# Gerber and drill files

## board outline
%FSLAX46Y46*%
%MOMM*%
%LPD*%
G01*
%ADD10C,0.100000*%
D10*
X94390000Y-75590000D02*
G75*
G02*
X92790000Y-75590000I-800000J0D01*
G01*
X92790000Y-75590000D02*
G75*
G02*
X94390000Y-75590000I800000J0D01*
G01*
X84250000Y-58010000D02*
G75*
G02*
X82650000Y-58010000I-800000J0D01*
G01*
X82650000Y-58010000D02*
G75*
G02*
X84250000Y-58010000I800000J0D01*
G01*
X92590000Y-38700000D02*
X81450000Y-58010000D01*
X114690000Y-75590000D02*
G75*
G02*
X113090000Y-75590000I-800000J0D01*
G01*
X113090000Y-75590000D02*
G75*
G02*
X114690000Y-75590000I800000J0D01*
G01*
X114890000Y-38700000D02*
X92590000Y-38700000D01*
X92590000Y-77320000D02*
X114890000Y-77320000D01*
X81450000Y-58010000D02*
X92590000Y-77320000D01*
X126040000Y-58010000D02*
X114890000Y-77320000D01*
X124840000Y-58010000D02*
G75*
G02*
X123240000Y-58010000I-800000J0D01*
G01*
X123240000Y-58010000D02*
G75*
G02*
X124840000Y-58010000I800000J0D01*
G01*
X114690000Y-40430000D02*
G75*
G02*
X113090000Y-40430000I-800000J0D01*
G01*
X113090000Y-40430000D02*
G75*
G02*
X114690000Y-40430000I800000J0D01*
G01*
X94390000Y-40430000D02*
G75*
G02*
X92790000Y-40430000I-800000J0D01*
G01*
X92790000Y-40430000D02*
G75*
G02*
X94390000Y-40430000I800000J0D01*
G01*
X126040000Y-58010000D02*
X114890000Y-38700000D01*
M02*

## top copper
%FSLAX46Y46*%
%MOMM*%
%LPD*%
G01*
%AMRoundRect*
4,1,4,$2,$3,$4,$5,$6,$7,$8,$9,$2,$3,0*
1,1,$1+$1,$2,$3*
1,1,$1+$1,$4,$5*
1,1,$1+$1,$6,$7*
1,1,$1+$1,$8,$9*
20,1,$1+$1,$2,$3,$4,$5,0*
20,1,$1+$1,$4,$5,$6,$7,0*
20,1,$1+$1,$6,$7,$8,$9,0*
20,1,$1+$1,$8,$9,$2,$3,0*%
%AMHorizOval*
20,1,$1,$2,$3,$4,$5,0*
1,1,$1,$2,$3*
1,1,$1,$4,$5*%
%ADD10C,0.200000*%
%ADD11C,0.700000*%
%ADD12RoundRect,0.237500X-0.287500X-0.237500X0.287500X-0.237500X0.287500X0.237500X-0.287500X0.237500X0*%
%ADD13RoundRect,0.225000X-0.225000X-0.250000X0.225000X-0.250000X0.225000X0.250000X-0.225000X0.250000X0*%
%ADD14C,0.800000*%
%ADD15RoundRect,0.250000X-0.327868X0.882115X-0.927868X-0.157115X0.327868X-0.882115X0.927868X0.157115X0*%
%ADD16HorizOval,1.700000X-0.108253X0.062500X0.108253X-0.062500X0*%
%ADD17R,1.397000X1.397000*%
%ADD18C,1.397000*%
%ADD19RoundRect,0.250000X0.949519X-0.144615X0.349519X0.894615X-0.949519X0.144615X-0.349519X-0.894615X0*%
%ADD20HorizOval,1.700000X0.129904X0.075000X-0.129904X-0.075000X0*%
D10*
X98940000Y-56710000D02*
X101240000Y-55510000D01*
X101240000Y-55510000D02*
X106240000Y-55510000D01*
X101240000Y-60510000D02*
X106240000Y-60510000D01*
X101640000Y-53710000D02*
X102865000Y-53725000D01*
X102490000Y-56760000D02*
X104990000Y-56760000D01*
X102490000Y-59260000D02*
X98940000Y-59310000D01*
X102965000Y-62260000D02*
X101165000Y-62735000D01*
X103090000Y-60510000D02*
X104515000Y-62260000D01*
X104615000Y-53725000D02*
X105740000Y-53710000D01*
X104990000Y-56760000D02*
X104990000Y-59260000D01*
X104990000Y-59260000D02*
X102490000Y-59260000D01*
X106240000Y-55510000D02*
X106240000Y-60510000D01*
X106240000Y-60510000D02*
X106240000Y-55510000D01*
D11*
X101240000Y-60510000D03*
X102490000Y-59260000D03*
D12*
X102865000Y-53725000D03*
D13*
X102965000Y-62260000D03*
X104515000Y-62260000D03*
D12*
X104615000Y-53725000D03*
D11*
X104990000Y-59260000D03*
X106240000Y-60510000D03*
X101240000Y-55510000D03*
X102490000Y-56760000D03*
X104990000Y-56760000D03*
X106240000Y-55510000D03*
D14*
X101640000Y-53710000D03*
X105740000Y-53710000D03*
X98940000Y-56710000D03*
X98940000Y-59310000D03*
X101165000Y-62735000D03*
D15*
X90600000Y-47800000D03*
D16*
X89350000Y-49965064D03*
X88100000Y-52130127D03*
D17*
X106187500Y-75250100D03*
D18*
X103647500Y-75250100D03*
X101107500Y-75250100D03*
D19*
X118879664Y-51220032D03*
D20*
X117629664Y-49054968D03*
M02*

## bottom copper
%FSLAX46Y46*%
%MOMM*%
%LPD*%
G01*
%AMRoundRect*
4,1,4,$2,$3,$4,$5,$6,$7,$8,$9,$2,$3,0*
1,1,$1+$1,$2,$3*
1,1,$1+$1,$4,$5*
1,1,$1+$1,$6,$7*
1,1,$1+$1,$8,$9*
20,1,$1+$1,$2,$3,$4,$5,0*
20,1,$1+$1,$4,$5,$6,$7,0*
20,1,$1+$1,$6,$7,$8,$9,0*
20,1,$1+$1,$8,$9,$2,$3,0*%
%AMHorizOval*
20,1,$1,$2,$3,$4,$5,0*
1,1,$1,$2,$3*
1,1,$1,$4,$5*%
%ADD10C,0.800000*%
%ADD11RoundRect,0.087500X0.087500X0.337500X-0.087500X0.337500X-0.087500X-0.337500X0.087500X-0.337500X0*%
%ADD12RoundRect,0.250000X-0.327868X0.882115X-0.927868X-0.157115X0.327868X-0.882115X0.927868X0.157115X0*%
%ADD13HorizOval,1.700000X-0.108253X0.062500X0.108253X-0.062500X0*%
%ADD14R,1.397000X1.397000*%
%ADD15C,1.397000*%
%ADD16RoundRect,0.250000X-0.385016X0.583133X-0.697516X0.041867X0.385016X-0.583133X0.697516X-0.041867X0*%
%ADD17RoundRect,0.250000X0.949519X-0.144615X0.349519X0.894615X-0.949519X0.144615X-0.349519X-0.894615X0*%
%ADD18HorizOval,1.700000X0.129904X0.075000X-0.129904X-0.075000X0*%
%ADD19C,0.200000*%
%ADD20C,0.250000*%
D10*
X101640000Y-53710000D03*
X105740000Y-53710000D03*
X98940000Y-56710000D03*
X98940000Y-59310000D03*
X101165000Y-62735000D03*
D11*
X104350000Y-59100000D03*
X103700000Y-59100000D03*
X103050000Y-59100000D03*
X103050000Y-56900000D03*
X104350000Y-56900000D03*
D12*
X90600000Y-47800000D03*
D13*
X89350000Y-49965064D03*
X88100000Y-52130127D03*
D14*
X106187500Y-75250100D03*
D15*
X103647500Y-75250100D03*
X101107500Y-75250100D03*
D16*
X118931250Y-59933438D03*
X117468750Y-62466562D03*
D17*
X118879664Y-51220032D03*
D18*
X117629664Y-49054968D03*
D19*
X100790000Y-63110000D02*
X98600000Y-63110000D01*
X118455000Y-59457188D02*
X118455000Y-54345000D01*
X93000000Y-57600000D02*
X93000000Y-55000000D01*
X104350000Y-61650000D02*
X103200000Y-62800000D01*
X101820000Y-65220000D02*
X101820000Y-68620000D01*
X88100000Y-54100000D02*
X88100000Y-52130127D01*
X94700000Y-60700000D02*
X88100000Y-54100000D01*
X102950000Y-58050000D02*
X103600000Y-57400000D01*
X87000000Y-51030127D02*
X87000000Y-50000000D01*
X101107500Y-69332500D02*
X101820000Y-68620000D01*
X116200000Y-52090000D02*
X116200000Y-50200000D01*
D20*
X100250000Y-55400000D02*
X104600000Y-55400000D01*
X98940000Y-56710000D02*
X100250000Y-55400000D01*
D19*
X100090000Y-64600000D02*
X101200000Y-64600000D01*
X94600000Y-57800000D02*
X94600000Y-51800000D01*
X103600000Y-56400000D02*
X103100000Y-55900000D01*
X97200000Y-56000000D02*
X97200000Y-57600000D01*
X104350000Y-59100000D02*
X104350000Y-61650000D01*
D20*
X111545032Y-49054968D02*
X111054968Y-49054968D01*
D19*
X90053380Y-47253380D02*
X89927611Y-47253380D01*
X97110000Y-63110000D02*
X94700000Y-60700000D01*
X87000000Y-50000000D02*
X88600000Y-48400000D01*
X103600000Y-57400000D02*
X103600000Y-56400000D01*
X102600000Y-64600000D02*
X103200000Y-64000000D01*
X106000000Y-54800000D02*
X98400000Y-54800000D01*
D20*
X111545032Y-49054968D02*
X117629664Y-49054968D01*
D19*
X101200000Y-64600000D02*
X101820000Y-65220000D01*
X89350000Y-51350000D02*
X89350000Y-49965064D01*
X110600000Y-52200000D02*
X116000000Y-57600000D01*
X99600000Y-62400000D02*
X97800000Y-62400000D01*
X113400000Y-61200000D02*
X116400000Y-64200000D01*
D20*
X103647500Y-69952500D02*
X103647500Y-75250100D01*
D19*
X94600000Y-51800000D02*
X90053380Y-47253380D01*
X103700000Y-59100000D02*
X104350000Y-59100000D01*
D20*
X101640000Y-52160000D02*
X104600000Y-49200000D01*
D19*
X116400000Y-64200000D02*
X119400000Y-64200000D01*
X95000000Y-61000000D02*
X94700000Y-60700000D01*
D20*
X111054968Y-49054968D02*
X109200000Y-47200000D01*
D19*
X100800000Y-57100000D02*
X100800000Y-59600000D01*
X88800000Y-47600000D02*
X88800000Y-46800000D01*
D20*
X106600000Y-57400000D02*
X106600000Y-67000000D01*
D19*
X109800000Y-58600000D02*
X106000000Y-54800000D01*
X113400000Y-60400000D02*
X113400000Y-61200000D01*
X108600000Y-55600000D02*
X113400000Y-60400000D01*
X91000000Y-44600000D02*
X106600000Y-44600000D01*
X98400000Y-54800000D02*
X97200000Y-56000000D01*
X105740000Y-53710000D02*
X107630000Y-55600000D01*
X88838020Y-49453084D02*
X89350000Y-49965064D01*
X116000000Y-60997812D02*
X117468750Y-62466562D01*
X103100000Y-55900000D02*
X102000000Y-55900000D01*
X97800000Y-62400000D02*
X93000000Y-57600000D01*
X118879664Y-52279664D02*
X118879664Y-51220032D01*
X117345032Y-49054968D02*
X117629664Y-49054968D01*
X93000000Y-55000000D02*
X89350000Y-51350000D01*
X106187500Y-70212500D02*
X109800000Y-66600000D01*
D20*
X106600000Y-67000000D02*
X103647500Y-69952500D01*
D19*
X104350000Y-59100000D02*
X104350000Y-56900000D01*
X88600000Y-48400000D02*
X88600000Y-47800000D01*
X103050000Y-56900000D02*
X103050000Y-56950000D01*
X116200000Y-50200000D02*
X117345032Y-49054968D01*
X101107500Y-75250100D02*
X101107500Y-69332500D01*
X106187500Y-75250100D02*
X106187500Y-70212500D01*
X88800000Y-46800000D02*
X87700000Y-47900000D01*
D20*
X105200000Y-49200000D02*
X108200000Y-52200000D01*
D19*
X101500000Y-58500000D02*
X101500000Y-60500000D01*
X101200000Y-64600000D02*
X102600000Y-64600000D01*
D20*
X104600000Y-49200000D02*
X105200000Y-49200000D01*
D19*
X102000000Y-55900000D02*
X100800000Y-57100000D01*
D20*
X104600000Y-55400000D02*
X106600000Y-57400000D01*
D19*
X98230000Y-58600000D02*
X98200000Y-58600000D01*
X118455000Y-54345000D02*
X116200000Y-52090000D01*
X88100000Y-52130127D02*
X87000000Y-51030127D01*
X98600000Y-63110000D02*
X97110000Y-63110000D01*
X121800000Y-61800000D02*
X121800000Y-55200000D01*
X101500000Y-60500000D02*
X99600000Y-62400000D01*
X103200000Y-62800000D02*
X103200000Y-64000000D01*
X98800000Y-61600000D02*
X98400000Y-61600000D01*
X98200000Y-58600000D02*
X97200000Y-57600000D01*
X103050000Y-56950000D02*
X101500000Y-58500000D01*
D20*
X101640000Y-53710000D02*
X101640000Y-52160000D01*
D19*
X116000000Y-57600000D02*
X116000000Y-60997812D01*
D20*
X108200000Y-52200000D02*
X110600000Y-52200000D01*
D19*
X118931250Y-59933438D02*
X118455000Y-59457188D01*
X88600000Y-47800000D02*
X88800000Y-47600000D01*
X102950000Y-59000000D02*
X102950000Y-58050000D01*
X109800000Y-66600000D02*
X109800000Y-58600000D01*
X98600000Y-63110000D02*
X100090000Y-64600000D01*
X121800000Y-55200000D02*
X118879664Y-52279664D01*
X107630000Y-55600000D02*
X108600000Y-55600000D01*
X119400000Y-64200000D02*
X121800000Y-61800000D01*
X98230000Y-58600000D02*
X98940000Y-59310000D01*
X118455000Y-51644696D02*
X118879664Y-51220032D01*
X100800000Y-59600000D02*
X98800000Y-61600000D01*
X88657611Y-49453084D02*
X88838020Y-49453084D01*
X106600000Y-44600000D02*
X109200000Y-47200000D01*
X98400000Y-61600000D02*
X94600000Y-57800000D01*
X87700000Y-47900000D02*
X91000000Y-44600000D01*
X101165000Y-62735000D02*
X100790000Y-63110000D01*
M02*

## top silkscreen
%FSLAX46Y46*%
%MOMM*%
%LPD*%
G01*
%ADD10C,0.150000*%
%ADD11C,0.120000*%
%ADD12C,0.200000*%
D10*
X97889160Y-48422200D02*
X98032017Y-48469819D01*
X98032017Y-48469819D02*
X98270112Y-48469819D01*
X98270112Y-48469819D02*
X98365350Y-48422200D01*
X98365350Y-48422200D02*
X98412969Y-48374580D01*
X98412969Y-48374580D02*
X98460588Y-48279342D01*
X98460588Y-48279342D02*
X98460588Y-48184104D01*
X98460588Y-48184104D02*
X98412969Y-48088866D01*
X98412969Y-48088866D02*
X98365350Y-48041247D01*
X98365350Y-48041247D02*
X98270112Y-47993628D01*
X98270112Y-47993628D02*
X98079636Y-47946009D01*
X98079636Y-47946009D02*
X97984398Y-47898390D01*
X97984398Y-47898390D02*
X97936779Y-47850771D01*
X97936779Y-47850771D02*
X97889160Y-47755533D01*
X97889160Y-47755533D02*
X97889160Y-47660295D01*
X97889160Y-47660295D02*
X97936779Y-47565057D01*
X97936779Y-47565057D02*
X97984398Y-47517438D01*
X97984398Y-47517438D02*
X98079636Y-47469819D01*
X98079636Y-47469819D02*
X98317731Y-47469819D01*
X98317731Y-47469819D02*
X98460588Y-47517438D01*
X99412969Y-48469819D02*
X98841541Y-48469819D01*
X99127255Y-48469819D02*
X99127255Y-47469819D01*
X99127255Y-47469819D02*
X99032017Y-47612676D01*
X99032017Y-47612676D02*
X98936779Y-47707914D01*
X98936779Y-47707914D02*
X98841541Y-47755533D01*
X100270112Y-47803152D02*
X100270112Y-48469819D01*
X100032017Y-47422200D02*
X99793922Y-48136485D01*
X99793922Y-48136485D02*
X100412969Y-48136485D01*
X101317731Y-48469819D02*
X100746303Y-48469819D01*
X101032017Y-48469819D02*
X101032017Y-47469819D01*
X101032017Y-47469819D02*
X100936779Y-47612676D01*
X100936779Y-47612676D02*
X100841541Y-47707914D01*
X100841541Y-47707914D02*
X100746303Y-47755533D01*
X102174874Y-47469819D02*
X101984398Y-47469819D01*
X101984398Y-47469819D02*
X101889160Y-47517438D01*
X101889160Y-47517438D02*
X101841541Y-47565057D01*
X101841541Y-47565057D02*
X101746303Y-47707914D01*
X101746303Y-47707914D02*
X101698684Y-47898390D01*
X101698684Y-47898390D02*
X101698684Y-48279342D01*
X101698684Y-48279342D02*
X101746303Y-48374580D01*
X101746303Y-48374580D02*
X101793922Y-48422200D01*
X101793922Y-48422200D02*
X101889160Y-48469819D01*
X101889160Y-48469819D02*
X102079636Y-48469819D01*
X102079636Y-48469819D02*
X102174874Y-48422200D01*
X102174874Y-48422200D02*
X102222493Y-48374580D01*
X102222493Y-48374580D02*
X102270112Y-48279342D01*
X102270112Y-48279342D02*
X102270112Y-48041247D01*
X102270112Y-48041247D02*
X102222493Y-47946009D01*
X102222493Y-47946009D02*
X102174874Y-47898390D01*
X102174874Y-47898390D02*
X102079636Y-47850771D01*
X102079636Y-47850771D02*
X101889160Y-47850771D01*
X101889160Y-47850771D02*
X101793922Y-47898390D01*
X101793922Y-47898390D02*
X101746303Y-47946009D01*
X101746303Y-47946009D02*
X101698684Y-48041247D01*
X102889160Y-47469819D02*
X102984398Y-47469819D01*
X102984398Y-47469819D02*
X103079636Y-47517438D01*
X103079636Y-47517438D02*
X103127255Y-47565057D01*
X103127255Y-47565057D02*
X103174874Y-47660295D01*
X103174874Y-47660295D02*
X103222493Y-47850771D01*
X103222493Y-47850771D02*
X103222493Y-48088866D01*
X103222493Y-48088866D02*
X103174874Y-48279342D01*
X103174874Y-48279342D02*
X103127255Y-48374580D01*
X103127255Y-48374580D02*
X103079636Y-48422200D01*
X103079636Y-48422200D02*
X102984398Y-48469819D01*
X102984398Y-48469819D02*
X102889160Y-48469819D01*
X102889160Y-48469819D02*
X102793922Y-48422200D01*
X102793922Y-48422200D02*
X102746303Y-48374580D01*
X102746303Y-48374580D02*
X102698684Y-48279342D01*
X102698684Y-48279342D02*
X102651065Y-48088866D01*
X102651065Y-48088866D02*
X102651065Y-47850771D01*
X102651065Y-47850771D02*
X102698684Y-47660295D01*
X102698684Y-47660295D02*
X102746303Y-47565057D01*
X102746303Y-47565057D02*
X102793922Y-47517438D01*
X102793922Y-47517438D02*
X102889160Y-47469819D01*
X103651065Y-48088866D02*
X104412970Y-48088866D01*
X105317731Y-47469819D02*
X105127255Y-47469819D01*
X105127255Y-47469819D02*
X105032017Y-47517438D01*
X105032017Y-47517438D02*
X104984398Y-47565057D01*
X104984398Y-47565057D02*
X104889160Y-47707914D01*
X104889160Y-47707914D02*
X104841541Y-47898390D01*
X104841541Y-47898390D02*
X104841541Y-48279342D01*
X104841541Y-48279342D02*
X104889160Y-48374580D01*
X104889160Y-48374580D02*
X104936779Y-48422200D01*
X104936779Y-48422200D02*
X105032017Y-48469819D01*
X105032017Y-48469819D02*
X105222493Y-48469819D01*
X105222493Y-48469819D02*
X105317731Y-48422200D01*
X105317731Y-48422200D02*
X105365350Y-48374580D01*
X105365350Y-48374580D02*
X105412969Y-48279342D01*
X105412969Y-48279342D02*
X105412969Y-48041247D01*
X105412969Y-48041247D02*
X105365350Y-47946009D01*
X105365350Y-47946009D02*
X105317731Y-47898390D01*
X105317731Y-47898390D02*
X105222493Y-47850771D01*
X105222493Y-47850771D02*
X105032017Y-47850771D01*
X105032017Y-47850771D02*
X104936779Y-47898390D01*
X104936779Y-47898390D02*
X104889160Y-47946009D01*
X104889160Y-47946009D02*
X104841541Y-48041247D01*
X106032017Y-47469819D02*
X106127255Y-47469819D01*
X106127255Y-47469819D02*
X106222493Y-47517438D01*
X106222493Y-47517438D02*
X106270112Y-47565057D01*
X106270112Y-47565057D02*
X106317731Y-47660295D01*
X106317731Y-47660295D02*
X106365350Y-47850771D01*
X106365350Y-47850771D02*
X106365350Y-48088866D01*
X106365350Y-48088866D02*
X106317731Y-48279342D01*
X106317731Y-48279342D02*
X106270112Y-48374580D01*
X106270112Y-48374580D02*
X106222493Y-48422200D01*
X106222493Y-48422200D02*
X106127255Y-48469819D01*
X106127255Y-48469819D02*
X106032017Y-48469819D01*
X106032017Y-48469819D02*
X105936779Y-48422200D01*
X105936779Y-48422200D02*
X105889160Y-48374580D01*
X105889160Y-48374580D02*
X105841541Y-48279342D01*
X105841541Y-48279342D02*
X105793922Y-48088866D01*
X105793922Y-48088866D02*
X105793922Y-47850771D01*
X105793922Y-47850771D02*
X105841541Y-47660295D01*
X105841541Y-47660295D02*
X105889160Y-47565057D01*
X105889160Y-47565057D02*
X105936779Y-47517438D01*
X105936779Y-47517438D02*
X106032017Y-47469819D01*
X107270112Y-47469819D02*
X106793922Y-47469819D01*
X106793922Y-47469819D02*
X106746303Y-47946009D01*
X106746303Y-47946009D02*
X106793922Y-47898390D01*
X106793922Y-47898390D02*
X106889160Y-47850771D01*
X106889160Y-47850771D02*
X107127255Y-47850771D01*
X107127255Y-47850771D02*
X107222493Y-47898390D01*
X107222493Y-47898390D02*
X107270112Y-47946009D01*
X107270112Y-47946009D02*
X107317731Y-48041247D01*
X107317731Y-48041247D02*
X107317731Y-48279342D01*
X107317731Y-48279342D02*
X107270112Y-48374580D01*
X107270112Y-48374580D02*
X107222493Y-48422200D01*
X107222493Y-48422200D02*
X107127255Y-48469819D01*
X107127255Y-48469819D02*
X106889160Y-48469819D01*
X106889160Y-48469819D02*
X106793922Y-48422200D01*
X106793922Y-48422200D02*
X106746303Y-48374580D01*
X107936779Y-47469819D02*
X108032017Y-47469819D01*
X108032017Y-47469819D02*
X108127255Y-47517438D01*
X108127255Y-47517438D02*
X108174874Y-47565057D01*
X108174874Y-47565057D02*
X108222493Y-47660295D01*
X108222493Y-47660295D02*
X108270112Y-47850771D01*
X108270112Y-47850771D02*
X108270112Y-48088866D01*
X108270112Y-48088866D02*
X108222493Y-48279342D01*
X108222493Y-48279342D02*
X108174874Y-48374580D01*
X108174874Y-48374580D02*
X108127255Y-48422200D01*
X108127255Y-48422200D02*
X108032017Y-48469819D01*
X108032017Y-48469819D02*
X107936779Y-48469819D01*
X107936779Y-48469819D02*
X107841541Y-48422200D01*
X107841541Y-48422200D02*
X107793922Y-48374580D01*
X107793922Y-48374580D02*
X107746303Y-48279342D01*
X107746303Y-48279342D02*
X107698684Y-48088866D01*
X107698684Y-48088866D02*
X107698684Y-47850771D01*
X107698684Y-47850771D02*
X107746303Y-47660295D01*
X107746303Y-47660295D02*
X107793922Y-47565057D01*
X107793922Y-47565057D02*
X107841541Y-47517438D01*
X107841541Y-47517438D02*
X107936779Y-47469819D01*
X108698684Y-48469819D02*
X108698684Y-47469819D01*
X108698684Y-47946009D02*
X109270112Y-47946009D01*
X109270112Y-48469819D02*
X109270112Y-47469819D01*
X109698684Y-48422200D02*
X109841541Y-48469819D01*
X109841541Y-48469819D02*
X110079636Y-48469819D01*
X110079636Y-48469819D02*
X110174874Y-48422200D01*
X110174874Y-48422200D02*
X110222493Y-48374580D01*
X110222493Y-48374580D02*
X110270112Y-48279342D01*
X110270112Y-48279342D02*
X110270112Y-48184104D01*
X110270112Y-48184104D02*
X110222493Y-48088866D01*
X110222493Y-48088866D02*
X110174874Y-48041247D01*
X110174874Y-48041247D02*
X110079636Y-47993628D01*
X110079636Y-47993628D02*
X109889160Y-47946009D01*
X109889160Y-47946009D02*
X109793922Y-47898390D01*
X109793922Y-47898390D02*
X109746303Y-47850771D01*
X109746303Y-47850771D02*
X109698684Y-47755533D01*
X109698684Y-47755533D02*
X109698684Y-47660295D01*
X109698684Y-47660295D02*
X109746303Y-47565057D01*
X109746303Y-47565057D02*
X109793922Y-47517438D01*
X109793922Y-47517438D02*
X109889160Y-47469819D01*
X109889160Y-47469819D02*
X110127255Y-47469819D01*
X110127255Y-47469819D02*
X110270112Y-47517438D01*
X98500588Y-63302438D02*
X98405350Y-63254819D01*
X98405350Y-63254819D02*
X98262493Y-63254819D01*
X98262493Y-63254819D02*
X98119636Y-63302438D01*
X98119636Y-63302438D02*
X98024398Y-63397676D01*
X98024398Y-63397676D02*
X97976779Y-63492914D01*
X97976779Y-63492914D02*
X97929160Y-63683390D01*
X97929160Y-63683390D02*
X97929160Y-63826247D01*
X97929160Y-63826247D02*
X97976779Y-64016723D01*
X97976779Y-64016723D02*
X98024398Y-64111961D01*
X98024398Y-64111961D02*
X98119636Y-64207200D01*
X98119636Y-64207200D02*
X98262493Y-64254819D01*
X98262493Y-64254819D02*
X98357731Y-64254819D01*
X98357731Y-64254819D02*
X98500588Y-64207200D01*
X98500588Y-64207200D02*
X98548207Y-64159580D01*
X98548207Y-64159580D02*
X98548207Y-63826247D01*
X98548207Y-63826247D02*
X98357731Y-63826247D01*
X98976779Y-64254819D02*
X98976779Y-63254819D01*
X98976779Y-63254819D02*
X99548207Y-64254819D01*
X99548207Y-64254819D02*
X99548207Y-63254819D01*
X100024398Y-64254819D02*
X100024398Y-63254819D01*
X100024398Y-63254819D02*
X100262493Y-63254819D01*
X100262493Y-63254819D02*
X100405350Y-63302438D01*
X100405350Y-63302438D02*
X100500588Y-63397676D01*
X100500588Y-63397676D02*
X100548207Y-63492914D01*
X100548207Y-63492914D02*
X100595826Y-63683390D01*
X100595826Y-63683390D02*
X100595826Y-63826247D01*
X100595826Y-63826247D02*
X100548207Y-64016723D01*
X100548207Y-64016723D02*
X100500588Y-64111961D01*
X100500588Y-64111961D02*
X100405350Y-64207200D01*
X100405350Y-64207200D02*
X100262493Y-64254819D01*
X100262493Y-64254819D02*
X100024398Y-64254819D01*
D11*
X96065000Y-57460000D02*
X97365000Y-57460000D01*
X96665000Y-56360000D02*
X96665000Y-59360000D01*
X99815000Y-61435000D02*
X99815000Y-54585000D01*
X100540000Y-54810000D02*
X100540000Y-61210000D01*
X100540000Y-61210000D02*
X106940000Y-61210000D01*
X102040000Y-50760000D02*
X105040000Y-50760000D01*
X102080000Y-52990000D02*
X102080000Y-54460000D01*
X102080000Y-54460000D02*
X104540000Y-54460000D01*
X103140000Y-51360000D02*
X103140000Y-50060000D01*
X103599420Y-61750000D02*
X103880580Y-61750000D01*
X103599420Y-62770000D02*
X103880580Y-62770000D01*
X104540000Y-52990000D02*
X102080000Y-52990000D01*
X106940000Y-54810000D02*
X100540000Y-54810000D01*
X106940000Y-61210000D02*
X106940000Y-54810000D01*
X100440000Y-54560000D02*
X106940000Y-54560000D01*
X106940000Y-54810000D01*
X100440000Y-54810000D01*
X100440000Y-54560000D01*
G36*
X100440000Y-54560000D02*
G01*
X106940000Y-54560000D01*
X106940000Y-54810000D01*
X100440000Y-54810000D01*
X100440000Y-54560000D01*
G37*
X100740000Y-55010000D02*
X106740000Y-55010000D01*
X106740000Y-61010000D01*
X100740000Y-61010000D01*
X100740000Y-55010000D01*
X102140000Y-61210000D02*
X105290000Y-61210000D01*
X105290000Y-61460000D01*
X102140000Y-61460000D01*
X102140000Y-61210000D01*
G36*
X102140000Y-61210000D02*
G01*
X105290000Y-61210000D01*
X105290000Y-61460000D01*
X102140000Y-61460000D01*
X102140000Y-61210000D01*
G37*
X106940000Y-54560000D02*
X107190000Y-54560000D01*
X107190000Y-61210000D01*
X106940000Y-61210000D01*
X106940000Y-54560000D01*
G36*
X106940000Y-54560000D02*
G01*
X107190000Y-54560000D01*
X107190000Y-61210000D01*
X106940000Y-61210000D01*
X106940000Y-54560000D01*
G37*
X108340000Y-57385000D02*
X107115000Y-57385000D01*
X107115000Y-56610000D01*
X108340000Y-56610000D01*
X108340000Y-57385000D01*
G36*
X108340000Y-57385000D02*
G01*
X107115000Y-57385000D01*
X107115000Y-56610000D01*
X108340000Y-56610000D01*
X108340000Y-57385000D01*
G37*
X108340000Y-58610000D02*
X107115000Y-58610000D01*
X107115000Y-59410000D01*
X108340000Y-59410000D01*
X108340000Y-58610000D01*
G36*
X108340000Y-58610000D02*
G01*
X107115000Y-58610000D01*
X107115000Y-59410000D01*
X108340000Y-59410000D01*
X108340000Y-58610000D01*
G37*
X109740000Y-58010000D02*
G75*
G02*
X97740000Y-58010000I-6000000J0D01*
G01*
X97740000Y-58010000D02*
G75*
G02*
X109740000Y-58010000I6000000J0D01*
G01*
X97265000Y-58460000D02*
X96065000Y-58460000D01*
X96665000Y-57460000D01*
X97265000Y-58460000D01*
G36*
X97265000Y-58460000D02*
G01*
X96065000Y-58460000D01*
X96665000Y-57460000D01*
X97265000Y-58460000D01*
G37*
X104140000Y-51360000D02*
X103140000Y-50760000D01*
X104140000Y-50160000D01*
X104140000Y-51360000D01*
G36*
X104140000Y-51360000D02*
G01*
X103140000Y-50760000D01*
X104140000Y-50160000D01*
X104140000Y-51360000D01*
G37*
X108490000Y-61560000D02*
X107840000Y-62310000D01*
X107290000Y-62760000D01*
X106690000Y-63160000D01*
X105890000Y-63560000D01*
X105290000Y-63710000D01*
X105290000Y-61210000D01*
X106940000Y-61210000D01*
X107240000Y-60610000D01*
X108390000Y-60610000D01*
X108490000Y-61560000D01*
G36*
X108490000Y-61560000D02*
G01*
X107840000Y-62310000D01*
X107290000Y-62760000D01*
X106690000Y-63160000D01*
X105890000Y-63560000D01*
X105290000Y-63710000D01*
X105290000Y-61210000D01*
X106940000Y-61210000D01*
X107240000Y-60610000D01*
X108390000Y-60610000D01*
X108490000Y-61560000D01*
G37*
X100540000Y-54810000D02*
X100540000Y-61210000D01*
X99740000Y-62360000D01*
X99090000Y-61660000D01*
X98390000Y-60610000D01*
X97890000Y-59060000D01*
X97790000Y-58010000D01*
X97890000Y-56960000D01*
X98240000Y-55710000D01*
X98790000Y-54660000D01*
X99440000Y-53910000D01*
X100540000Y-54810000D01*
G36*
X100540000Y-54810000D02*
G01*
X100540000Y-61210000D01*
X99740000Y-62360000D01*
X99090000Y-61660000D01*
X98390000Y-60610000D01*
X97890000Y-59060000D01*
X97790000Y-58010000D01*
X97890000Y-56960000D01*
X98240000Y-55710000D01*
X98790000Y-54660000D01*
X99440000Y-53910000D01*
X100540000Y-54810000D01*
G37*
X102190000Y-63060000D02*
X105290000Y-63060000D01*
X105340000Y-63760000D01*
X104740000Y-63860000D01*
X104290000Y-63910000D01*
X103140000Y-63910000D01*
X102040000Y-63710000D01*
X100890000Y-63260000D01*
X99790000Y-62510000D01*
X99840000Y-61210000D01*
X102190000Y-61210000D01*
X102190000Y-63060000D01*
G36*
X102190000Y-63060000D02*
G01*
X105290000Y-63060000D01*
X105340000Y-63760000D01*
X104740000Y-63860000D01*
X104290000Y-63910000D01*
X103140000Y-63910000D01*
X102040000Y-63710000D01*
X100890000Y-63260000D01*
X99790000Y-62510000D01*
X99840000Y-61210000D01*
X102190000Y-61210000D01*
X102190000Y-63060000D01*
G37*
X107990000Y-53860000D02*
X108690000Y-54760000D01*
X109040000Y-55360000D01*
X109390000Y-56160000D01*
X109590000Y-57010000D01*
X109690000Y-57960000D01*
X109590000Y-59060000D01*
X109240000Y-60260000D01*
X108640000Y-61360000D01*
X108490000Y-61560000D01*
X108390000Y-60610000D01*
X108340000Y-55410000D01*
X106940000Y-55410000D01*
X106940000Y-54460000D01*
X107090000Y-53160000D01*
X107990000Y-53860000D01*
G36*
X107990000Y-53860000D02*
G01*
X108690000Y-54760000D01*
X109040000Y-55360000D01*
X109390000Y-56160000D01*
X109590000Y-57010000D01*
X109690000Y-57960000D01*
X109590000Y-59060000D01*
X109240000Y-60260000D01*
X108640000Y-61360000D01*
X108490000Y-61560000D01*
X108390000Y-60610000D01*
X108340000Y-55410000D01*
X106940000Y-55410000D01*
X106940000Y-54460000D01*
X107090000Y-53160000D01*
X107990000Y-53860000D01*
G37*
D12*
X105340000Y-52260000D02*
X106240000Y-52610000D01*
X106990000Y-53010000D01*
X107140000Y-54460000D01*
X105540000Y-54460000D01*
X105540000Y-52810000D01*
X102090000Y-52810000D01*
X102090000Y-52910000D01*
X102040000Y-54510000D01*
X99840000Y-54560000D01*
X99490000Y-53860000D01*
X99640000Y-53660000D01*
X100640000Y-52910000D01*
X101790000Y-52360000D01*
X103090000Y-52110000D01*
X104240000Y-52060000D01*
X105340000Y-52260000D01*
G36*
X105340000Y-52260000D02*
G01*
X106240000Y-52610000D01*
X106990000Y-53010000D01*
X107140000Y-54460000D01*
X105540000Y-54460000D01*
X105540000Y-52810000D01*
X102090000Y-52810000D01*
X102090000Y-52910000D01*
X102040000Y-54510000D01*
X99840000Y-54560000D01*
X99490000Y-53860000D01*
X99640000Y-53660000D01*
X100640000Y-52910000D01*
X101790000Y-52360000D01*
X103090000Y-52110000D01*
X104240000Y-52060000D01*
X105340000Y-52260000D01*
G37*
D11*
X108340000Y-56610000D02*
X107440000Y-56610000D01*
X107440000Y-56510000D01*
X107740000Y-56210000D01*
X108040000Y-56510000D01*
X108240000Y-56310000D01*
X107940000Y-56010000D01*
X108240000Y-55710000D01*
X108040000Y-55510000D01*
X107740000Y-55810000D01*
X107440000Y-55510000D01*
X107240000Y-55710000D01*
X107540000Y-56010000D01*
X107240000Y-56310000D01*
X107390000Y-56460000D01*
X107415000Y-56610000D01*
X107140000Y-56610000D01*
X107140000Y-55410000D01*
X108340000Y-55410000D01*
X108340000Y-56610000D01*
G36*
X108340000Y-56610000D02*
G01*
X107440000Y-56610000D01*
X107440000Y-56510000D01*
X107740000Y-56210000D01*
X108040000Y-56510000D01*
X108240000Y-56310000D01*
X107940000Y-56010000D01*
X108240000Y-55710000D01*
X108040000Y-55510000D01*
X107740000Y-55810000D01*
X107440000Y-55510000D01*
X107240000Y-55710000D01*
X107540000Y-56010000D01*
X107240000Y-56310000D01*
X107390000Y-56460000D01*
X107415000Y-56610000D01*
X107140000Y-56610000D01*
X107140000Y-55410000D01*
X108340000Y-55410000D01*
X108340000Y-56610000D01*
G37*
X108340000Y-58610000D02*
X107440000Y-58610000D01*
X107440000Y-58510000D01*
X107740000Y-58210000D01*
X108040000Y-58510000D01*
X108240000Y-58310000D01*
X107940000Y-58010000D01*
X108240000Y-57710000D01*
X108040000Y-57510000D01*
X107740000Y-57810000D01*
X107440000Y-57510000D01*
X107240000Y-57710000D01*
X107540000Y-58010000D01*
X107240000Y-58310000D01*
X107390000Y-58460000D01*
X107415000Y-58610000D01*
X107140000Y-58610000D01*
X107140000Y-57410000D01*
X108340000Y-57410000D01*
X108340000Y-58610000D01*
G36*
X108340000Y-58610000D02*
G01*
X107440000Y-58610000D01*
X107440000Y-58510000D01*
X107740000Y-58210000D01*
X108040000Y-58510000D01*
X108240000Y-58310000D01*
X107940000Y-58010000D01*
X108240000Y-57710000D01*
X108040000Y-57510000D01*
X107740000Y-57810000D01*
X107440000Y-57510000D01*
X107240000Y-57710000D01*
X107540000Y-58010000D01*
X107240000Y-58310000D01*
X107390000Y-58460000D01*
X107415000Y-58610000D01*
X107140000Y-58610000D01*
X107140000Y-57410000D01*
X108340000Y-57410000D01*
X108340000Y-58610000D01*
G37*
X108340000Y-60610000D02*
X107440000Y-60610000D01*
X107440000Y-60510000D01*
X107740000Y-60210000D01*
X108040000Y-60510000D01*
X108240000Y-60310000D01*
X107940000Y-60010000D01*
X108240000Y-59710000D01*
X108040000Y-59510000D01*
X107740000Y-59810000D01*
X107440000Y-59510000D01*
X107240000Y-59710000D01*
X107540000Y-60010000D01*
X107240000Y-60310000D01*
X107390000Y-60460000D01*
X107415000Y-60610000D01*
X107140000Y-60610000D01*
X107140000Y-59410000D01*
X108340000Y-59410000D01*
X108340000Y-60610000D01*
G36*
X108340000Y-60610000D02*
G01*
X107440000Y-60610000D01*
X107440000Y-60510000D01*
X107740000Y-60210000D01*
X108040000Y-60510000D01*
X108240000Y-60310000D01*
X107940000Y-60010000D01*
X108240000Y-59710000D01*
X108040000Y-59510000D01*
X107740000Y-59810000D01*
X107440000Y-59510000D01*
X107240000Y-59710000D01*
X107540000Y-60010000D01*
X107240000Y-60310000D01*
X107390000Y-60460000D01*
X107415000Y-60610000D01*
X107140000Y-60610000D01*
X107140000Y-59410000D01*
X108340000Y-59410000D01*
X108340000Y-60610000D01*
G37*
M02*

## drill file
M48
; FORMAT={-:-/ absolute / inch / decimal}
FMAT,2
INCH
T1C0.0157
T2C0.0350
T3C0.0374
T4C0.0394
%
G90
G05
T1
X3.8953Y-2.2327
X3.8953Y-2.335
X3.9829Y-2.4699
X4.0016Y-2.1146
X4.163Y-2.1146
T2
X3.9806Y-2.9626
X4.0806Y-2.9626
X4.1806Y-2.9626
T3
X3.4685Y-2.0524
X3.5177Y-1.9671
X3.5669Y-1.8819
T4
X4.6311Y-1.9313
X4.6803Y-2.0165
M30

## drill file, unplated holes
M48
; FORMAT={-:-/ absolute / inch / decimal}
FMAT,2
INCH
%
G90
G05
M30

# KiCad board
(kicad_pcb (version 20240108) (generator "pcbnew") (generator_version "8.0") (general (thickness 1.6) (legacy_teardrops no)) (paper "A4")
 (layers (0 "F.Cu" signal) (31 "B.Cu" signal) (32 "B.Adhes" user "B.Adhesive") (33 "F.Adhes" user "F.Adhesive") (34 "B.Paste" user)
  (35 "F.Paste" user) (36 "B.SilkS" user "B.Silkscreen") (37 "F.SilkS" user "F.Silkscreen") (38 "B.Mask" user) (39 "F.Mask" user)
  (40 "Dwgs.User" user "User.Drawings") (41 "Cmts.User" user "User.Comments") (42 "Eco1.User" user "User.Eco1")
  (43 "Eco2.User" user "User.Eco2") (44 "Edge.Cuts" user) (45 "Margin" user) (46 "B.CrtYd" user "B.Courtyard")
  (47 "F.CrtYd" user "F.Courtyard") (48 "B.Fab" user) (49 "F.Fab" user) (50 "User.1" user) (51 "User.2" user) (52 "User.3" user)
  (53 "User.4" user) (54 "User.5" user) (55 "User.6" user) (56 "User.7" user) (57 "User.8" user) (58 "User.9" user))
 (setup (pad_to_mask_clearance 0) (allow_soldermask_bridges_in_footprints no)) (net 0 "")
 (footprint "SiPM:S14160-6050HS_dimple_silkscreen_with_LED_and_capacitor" (layer "F.Cu") (at 103.74 58.01)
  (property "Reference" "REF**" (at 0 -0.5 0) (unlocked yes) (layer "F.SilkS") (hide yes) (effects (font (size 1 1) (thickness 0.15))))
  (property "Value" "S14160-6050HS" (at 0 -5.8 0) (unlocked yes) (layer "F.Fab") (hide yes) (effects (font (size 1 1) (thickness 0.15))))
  (fp_line (start -4.8 -1.3) (end -2.5 -2.5) (stroke (width 0.2) (type default)) (layer "F.Cu"))
  (fp_line (start -2.5 -2.5) (end 2.5 -2.5) (stroke (width 0.2) (type default)) (layer "F.Cu"))
  (fp_line (start -2.5 2.5) (end 2.5 2.5) (stroke (width 0.2) (type default)) (layer "F.Cu"))
  (fp_line (start -2.1 -4.3) (end -0.875 -4.285) (stroke (width 0.2) (type default)) (layer "F.Cu"))
  (fp_line (start -1.25 -1.25) (end 1.25 -1.25) (stroke (width 0.2) (type default)) (layer "F.Cu"))
  (fp_line (start -1.25 1.25) (end -4.8 1.3) (stroke (width 0.2) (type default)) (layer "F.Cu"))
  (fp_line (start -0.775 4.25) (end -2.575 4.725) (stroke (width 0.2) (type default)) (layer "F.Cu"))
  (fp_line (start -0.65 2.5) (end 0.775 4.25) (stroke (width 0.2) (type default)) (layer "F.Cu"))
  (fp_line (start 0.875 -4.285) (end 2 -4.3) (stroke (width 0.2) (type default)) (layer "F.Cu"))
  (fp_line (start 1.25 -1.25) (end 1.25 1.25) (stroke (width 0.2) (type default)) (layer "F.Cu"))
  (fp_line (start 1.25 1.25) (end -1.25 1.25) (stroke (width 0.2) (type default)) (layer "F.Cu"))
  (fp_line (start 2.5 -2.5) (end 2.5 2.5) (stroke (width 0.2) (type default)) (layer "F.Cu"))
  (fp_line (start 2.5 2.5) (end 2.5 -2.5) (stroke (width 0.2) (type default)) (layer "F.Cu"))
  (fp_line (start -7.675 -0.55) (end -6.375 -0.55) (stroke (width 0.12) (type solid)) (layer "F.SilkS"))
  (fp_line (start -7.075 -1.65) (end -7.075 1.35) (stroke (width 0.12) (type solid)) (layer "F.SilkS"))
  (fp_line (start -3.925 3.425) (end -3.925 -3.425) (stroke (width 0.12) (type solid)) (layer "F.SilkS"))
  (fp_line (start -3.2 -3.2) (end -3.2 3.2) (stroke (width 0.12) (type default)) (layer "F.SilkS"))
  (fp_line (start -3.2 3.2) (end 3.2 3.2) (stroke (width 0.12) (type solid)) (layer "F.SilkS"))
  (fp_line (start -1.7 -7.25) (end 1.3 -7.25) (stroke (width 0.12) (type solid)) (layer "F.SilkS"))
  (fp_line (start -1.66 -5.02) (end -1.66 -3.55) (stroke (width 0.12) (type solid)) (layer "F.SilkS"))
  (fp_line (start -1.66 -3.55) (end 0.8 -3.55) (stroke (width 0.12) (type solid)) (layer "F.SilkS"))
  (fp_line (start -0.6 -6.65) (end -0.6 -7.95) (stroke (width 0.12) (type solid)) (layer "F.SilkS"))
  (fp_line (start -0.14058 3.74) (end 0.14058 3.74) (stroke (width 0.12) (type solid)) (layer "F.SilkS"))
  (fp_line (start -0.14058 4.76) (end 0.14058 4.76) (stroke (width 0.12) (type solid)) (layer "F.SilkS"))
  (fp_line (start 0.8 -5.02) (end -1.66 -5.02) (stroke (width 0.12) (type solid)) (layer "F.SilkS"))
  (fp_line (start 3.2 -3.2) (end -3.2 -3.2) (stroke (width 0.12) (type default)) (layer "F.SilkS"))
  (fp_line (start 3.2 3.2) (end 3.2 -3.2) (stroke (width 0.12) (type default)) (layer "F.SilkS"))
  (fp_rect (start -3.3 -3.45) (end 3.2 -3.2) (stroke (width 0.12) (type solid)) (fill solid) (layer "F.SilkS"))
  (fp_rect (start -3 -3) (end 3 3) (stroke (width 0.12) (type solid)) (fill none) (layer "F.SilkS"))
  (fp_rect (start -1.6 3.2) (end 1.55 3.45) (stroke (width 0.12) (type solid)) (fill solid) (layer "F.SilkS"))
  (fp_rect (start 3.2 -3.45) (end 3.45 3.2) (stroke (width 0.12) (type solid)) (fill solid) (layer "F.SilkS"))
  (fp_rect (start 4.6 -0.625) (end 3.375 -1.4) (stroke (width 0.12) (type solid)) (fill solid) (layer "F.SilkS"))
  (fp_rect (start 4.6 0.6) (end 3.375 1.4) (stroke (width 0.12) (type solid)) (fill solid) (layer "F.SilkS"))
  (fp_circle (center 0 0) (end 6 0) (stroke (width 0.12) (type solid)) (fill none) (layer "F.SilkS"))
  (fp_poly (pts (xy -7.075 -0.55) (xy -7.675 0.45) (xy -6.475 0.45)) (stroke (width 0.12) (type solid)) (fill solid) (layer "F.SilkS"))
  (fp_poly (pts (xy -0.6 -7.25) (xy 0.4 -6.65) (xy 0.4 -7.85)) (stroke (width 0.12) (type solid)) (fill solid) (layer "F.SilkS"))
  (fp_poly
   (pts (xy 1.55 3.2) (xy 1.55 5.7) (xy 2.15 5.55) (xy 2.95 5.15) (xy 3.55 4.75) (xy 4.1 4.3) (xy 4.75 3.55) (xy 4.65 2.6) (xy 3.5 2.6)
    (xy 3.2 3.2))
   (stroke (width 0.12) (type solid)) (fill solid) (layer "F.SilkS"))
  (fp_poly
   (pts (xy -4 4.35) (xy -4.65 3.65) (xy -5.35 2.6) (xy -5.85 1.05) (xy -5.95 0) (xy -5.85 -1.05) (xy -5.5 -2.3) (xy -4.95 -3.35)
    (xy -4.3 -4.1) (xy -3.2 -3.2) (xy -3.2 3.2))
   (stroke (width 0.12) (type solid)) (fill solid) (layer "F.SilkS"))
  (fp_poly
   (pts (xy 1.55 5.05) (xy -1.55 5.05) (xy -1.55 3.2) (xy -3.9 3.2) (xy -3.95 4.5) (xy -2.85 5.25) (xy -1.7 5.7) (xy -0.6 5.9) (xy 0.55 5.9)
    (xy 1 5.85) (xy 1.6 5.75))
   (stroke (width 0.12) (type solid)) (fill solid) (layer "F.SilkS"))
  (fp_poly
   (pts (xy 3.2 -3.55) (xy 3.35 -4.85) (xy 4.25 -4.15) (xy 4.95 -3.25) (xy 5.3 -2.65) (xy 5.65 -1.85) (xy 5.85 -1) (xy 5.95 -0.05)
    (xy 5.85 1.05) (xy 5.5 2.25) (xy 4.9 3.35) (xy 4.75 3.55) (xy 4.65 2.6) (xy 4.6 -2.6) (xy 3.2 -2.6))
   (stroke (width 0.12) (type solid)) (fill solid) (layer "F.SilkS"))
  (fp_poly
   (pts (xy -3.9 -3.45) (xy -1.7 -3.5) (xy -1.65 -5.1) (xy -1.65 -5.2) (xy 1.8 -5.2) (xy 1.8 -3.55) (xy 3.4 -3.55) (xy 3.25 -5)
    (xy 2.5 -5.4) (xy 1.6 -5.75) (xy 0.5 -5.95) (xy -0.65 -5.9) (xy -1.95 -5.65) (xy -3.1 -5.1) (xy -4.1 -4.35) (xy -4.25 -4.15))
   (stroke (width 0.2) (type solid)) (fill solid) (layer "F.SilkS"))
  (fp_poly
   (pts (xy 4.6 -1.4) (xy 3.7 -1.4) (xy 3.7 -1.5) (xy 4 -1.8) (xy 4.3 -1.5) (xy 4.5 -1.7) (xy 4.2 -2) (xy 4.5 -2.3) (xy 4.3 -2.5)
    (xy 4 -2.2) (xy 3.7 -2.5) (xy 3.5 -2.3) (xy 3.8 -2) (xy 3.5 -1.7) (xy 3.65 -1.55) (xy 3.675 -1.4) (xy 3.4 -1.4) (xy 3.4 -2.6)
    (xy 4.6 -2.6))
   (stroke (width 0.12) (type solid)) (fill solid) (layer "F.SilkS"))
  (fp_poly
   (pts (xy 4.6 0.6) (xy 3.7 0.6) (xy 3.7 0.5) (xy 4 0.2) (xy 4.3 0.5) (xy 4.5 0.3) (xy 4.2 0) (xy 4.5 -0.3) (xy 4.3 -0.5) (xy 4 -0.2)
    (xy 3.7 -0.5) (xy 3.5 -0.3) (xy 3.8 0) (xy 3.5 0.3) (xy 3.65 0.45) (xy 3.675 0.6) (xy 3.4 0.6) (xy 3.4 -0.6) (xy 4.6 -0.6))
   (stroke (width 0.12) (type solid)) (fill solid) (layer "F.SilkS"))
  (fp_poly
   (pts (xy 4.6 2.6) (xy 3.7 2.6) (xy 3.7 2.5) (xy 4 2.2) (xy 4.3 2.5) (xy 4.5 2.3) (xy 4.2 2) (xy 4.5 1.7) (xy 4.3 1.5) (xy 4 1.8)
    (xy 3.7 1.5) (xy 3.5 1.7) (xy 3.8 2) (xy 3.5 2.3) (xy 3.65 2.45) (xy 3.675 2.6) (xy 3.4 2.6) (xy 3.4 1.4) (xy 4.6 1.4))
   (stroke (width 0.12) (type solid)) (fill solid) (layer "F.SilkS"))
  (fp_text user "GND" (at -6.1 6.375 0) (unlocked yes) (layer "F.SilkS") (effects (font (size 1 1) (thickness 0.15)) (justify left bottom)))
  (pad "1" smd circle (at -2.5 2.5) (size 0.7 0.7) (layers "F.Cu" "F.Paste" "F.Mask"))
  (pad "1" smd circle (at -1.25 1.25) (size 0.7 0.7) (layers "F.Cu" "F.Paste" "F.Mask"))
  (pad "1" smd roundrect (at -0.875 -4.285) (size 1.05 0.95) (layers "F.Cu" "F.Paste" "F.Mask") (roundrect_rratio 0.25))
  (pad "1" smd roundrect (at -0.775 4.25) (size 0.9 0.95) (layers "F.Cu" "F.Paste" "F.Mask") (roundrect_rratio 0.25))
  (pad "2" smd roundrect (at 0.775 4.25) (size 0.9 0.95) (layers "F.Cu" "F.Paste" "F.Mask") (roundrect_rratio 0.25))
  (pad "2" smd roundrect (at 0.875 -4.285) (size 1.05 0.95) (layers "F.Cu" "F.Paste" "F.Mask") (roundrect_rratio 0.25))
  (pad "2" smd circle (at 1.25 1.25) (size 0.7 0.7) (layers "F.Cu" "F.Paste" "F.Mask"))
  (pad "2" smd circle (at 2.5 2.5) (size 0.7 0.7) (layers "F.Cu" "F.Paste" "F.Mask"))
  (pad "3" smd circle (at -2.5 -2.5) (size 0.7 0.7) (layers "F.Cu" "F.Paste" "F.Mask"))
  (pad "3" smd circle (at -1.25 -1.25) (size 0.7 0.7) (layers "F.Cu" "F.Paste" "F.Mask"))
  (pad "4" smd circle (at 1.25 -1.25) (size 0.7 0.7) (layers "F.Cu" "F.Paste" "F.Mask"))
  (pad "4" smd circle (at 2.5 -2.5) (size 0.7 0.7) (layers "F.Cu" "F.Paste" "F.Mask"))
  (pad "5" thru_hole circle (at -2.1 -4.3) (size 0.8 0.8) (drill 0.4) (layers "*.Cu") (remove_unused_layers no))
  (pad "6" thru_hole circle (at 2 -4.3) (size 0.8 0.8) (drill 0.4) (layers "*.Cu") (remove_unused_layers no))
  (pad "7" thru_hole circle (at -4.8 -1.3) (size 0.8 0.8) (drill 0.4) (layers "*.Cu") (remove_unused_layers no))
  (pad "8" thru_hole circle (at -4.8 1.3) (size 0.8 0.8) (drill 0.4) (layers "*.Cu") (remove_unused_layers no))
  (pad "9" thru_hole circle (at -2.575 4.725) (size 0.8 0.8) (drill 0.4) (layers "*.Cu") (remove_unused_layers no)))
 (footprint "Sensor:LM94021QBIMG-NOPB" (layer "B.Cu") (at 103.7 58 180)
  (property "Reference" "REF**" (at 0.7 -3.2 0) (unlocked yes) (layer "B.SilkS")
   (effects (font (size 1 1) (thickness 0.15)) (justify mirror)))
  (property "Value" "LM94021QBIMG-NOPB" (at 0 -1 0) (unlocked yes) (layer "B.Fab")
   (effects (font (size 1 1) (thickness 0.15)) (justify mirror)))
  (pad "1" smd roundrect (at -0.65 -1.1 180) (size 0.35 0.85) (layers "B.Cu" "B.Paste" "B.Mask") (roundrect_rratio 0.25))
  (pad "2" smd roundrect (at 0 -1.1 180) (size 0.35 0.85) (layers "B.Cu" "B.Paste" "B.Mask") (roundrect_rratio 0.25))
  (pad "3" smd roundrect (at 0.65 -1.1 180) (size 0.35 0.85) (layers "B.Cu" "B.Paste" "B.Mask") (roundrect_rratio 0.25))
  (pad "4" smd roundrect (at 0.65 1.1 180) (size 0.35 0.85) (layers "B.Cu" "B.Paste" "B.Mask") (roundrect_rratio 0.25))
  (pad "5" smd roundrect (at -0.65 1.1 180) (size 0.35 0.85) (layers "B.Cu" "B.Paste" "B.Mask") (roundrect_rratio 0.25)))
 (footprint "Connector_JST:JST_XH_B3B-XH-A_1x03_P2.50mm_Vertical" (layer "B.Cu") (at 90.6 47.8 -120)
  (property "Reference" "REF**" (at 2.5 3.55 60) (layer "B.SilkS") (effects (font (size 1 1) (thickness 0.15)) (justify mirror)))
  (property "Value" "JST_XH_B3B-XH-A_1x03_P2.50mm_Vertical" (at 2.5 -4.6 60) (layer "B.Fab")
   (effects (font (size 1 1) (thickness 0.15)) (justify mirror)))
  (pad "1" thru_hole roundrect (at 0 0 240) (size 1.7 1.95) (drill 0.95) (layers "*.Cu" "*.Mask") (remove_unused_layers no)
   (roundrect_rratio 0.1470588235))
  (pad "2" thru_hole oval (at 2.5 0 240) (size 1.7 1.95) (drill 0.95) (layers "*.Cu" "*.Mask") (remove_unused_layers no))
  (pad "3" thru_hole oval (at 5 0 240) (size 1.7 1.95) (drill 0.95) (layers "*.Cu" "*.Mask") (remove_unused_layers no)))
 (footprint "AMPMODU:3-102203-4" (layer "B.Cu") (at 106.1875 75.2501 180)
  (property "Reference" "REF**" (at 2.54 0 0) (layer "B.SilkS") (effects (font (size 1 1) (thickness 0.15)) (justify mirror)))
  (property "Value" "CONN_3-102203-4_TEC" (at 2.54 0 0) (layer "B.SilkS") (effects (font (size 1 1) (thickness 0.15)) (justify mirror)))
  (pad "1" thru_hole rect (at 0 0 180) (size 1.397 1.397) (drill 0.889) (layers "*.Cu" "*.Mask") (remove_unused_layers no))
  (pad "2" thru_hole circle (at 2.54 0 180) (size 1.397 1.397) (drill 0.889) (layers "*.Cu" "*.Mask") (remove_unused_layers no))
  (pad "3" thru_hole circle (at 5.08 0 180) (size 1.397 1.397) (drill 0.889) (layers "*.Cu" "*.Mask") (remove_unused_layers no)))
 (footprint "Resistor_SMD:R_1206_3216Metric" (layer "B.Cu") (at 118.2 61.2 -120)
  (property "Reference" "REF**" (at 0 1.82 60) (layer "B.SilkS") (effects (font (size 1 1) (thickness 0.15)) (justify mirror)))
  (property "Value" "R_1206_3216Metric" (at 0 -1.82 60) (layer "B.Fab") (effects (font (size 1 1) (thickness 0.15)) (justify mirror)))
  (pad "1" smd roundrect (at -1.4625 0 240) (size 1.125 1.75) (layers "B.Cu" "B.Paste" "B.Mask") (roundrect_rratio 0.222222))
  (pad "2" smd roundrect (at 1.4625 0 240) (size 1.125 1.75) (layers "B.Cu" "B.Paste" "B.Mask") (roundrect_rratio 0.222222)))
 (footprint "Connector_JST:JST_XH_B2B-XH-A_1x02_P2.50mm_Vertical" (layer "B.Cu") (at 118.879664 51.220032 120)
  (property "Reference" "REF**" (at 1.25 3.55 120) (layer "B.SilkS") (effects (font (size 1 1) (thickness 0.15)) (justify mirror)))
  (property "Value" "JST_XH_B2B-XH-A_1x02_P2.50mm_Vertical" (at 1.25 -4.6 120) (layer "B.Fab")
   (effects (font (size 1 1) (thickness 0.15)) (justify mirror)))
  (pad "1" thru_hole roundrect (at 0 0 120) (size 1.7 2) (drill 1) (layers "*.Cu" "*.Mask") (remove_unused_layers no)
   (roundrect_rratio 0.1470588235))
  (pad "2" thru_hole oval (at 2.5 0 120) (size 1.7 2) (drill 1) (layers "*.Cu" "*.Mask") (remove_unused_layers no)))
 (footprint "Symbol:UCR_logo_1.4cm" (layer "B.Cu") (at 104.4 43 180)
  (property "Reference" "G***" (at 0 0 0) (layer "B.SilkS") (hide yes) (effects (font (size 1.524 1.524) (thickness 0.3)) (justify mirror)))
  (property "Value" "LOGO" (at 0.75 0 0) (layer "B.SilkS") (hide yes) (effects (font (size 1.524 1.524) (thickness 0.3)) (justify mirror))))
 (gr_circle (center 93.59 75.59) (end 94.39 75.59) (stroke (width 0.1) (type solid)) (fill none) (layer "Edge.Cuts"))
 (gr_circle (center 83.45 58.01) (end 84.25 58.01) (stroke (width 0.1) (type solid)) (fill none) (layer "Edge.Cuts"))
 (gr_line (start 92.59 38.7) (end 81.45 58.01) (stroke (width 0.1) (type solid)) (layer "Edge.Cuts"))
 (gr_circle (center 113.89 75.59) (end 114.69 75.59) (stroke (width 0.1) (type solid)) (fill none) (layer "Edge.Cuts"))
 (gr_line (start 114.89 38.7) (end 92.59 38.7) (stroke (width 0.1) (type solid)) (layer "Edge.Cuts"))
 (gr_line (start 92.59 77.32) (end 114.89 77.32) (stroke (width 0.1) (type solid)) (layer "Edge.Cuts"))
 (gr_line (start 81.45 58.01) (end 92.59 77.32) (stroke (width 0.1) (type solid)) (layer "Edge.Cuts"))
 (gr_line (start 126.04 58.01) (end 114.89 77.32) (stroke (width 0.1) (type solid)) (layer "Edge.Cuts"))
 (gr_circle (center 124.04 58.01) (end 124.84 58.01) (stroke (width 0.1) (type solid)) (fill none) (layer "Edge.Cuts"))
 (gr_circle (center 113.89 40.43) (end 114.69 40.43) (stroke (width 0.1) (type solid)) (fill none) (layer "Edge.Cuts"))
 (gr_circle (center 93.59 40.43) (end 94.39 40.43) (stroke (width 0.1) (type solid)) (fill none) (layer "Edge.Cuts"))
 (gr_line (start 126.04 58.01) (end 114.89 38.7) (stroke (width 0.1) (type solid)) (layer "Edge.Cuts"))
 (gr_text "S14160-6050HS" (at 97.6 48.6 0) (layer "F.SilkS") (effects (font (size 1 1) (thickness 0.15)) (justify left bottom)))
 (segment (start 100.79 63.11) (end 98.6 63.11) (width 0.2) (layer "B.Cu") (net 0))
 (segment (start 118.455 59.457188) (end 118.455 54.345) (width 0.2) (layer "B.Cu") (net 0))
 (segment (start 93 57.6) (end 93 55) (width 0.2) (layer "B.Cu") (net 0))
 (segment (start 104.35 61.65) (end 103.2 62.8) (width 0.2) (layer "B.Cu") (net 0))
 (segment (start 101.82 65.22) (end 101.82 68.62) (width 0.2) (layer "B.Cu") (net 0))
 (segment (start 88.1 54.1) (end 88.1 52.130127) (width 0.2) (layer "B.Cu") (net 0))
 (segment (start 94.7 60.7) (end 88.1 54.1) (width 0.2) (layer "B.Cu") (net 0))
 (segment (start 102.95 58.05) (end 103.6 57.4) (width 0.2) (layer "B.Cu") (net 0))
 (segment (start 87 51.030127) (end 87 50) (width 0.2) (layer "B.Cu") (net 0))
 (segment (start 101.1075 69.3325) (end 101.82 68.62) (width 0.2) (layer "B.Cu") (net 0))
 (segment (start 116.2 52.09) (end 116.2 50.2) (width 0.2) (layer "B.Cu") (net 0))
 (segment (start 100.25 55.4) (end 104.6 55.4) (width 0.25) (layer "B.Cu") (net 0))
 (segment (start 98.94 56.71) (end 100.25 55.4) (width 0.25) (layer "B.Cu") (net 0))
 (segment (start 100.09 64.6) (end 101.2 64.6) (width 0.2) (layer "B.Cu") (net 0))
 (segment (start 94.6 57.8) (end 94.6 51.8) (width 0.2) (layer "B.Cu") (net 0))
 (segment (start 103.6 56.4) (end 103.1 55.9) (width 0.2) (layer "B.Cu") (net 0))
 (segment (start 97.2 56) (end 97.2 57.6) (width 0.2) (layer "B.Cu") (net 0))
 (segment (start 104.35 59.1) (end 104.35 61.65) (width 0.2) (layer "B.Cu") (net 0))
 (segment (start 111.545032 49.054968) (end 111.054968 49.054968) (width 0.25) (layer "B.Cu") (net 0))
 (segment (start 90.05338 47.25338) (end 89.927611 47.25338) (width 0.2) (layer "B.Cu") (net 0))
 (segment (start 97.11 63.11) (end 94.7 60.7) (width 0.2) (layer "B.Cu") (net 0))
 (segment (start 87 50) (end 88.6 48.4) (width 0.2) (layer "B.Cu") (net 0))
 (segment (start 103.6 57.4) (end 103.6 56.4) (width 0.2) (layer "B.Cu") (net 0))
 (segment (start 102.6 64.6) (end 103.2 64) (width 0.2) (layer "B.Cu") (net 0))
 (segment (start 106 54.8) (end 98.4 54.8) (width 0.2) (layer "B.Cu") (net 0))
 (segment (start 111.545032 49.054968) (end 117.629664 49.054968) (width 0.25) (layer "B.Cu") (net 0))
 (segment (start 101.2 64.6) (end 101.82 65.22) (width 0.2) (layer "B.Cu") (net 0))
 (segment (start 89.35 51.35) (end 89.35 49.965064) (width 0.2) (layer "B.Cu") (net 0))
 (segment (start 110.6 52.2) (end 116 57.6) (width 0.2) (layer "B.Cu") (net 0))
 (segment (start 99.6 62.4) (end 97.8 62.4) (width 0.2) (layer "B.Cu") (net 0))
 (segment (start 113.4 61.2) (end 116.4 64.2) (width 0.2) (layer "B.Cu") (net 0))
 (segment (start 103.6475 69.9525) (end 103.6475 75.2501) (width 0.25) (layer "B.Cu") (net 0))
 (segment (start 94.6 51.8) (end 90.05338 47.25338) (width 0.2) (layer "B.Cu") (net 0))
 (segment (start 103.7 59.1) (end 104.35 59.1) (width 0.2) (layer "B.Cu") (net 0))
 (segment (start 101.64 52.16) (end 104.6 49.2) (width 0.25) (layer "B.Cu") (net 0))
 (segment (start 116.4 64.2) (end 119.4 64.2) (width 0.2) (layer "B.Cu") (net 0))
 (segment (start 95 61) (end 94.7 60.7) (width 0.2) (layer "B.Cu") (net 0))
 (segment (start 111.054968 49.054968) (end 109.2 47.2) (width 0.25) (layer "B.Cu") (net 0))
 (segment (start 100.8 57.1) (end 100.8 59.6) (width 0.2) (layer "B.Cu") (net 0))
 (segment (start 88.8 47.6) (end 88.8 46.8) (width 0.2) (layer "B.Cu") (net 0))
 (segment (start 106.6 57.4) (end 106.6 67) (width 0.25) (layer "B.Cu") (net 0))
 (segment (start 109.8 58.6) (end 106 54.8) (width 0.2) (layer "B.Cu") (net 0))
 (segment (start 113.4 60.4) (end 113.4 61.2) (width 0.2) (layer "B.Cu") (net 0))
 (segment (start 108.6 55.6) (end 113.4 60.4) (width 0.2) (layer "B.Cu") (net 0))
 (segment (start 91 44.6) (end 106.6 44.6) (width 0.2) (layer "B.Cu") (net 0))
 (segment (start 98.4 54.8) (end 97.2 56) (width 0.2) (layer "B.Cu") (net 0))
 (segment (start 105.74 53.71) (end 107.63 55.6) (width 0.2) (layer "B.Cu") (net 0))
 (segment (start 88.83802 49.453084) (end 89.35 49.965064) (width 0.2) (layer "B.Cu") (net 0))
 (segment (start 116 60.997812) (end 117.46875 62.466562) (width 0.2) (layer "B.Cu") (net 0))
 (segment (start 103.1 55.9) (end 102 55.9) (width 0.2) (layer "B.Cu") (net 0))
 (segment (start 97.8 62.4) (end 93 57.6) (width 0.2) (layer "B.Cu") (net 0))
 (segment (start 118.879664 52.279664) (end 118.879664 51.220032) (width 0.2) (layer "B.Cu") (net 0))
 (segment (start 117.345032 49.054968) (end 117.629664 49.054968) (width 0.2) (layer "B.Cu") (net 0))
 (segment (start 93 55) (end 89.35 51.35) (width 0.2) (layer "B.Cu") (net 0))
 (segment (start 106.1875 70.2125) (end 109.8 66.6) (width 0.2) (layer "B.Cu") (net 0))
 (segment (start 106.6 67) (end 103.6475 69.9525) (width 0.25) (layer "B.Cu") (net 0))
 (segment (start 104.35 59.1) (end 104.35 56.9) (width 0.2) (layer "B.Cu") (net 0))
 (segment (start 88.6 48.4) (end 88.6 47.8) (width 0.2) (layer "B.Cu") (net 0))
 (segment (start 103.05 56.9) (end 103.05 56.95) (width 0.2) (layer "B.Cu") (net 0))
 (segment (start 116.2 50.2) (end 117.345032 49.054968) (width 0.2) (layer "B.Cu") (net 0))
 (segment (start 101.1075 75.2501) (end 101.1075 69.3325) (width 0.2) (layer "B.Cu") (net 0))
 (segment (start 106.1875 75.2501) (end 106.1875 70.2125) (width 0.2) (layer "B.Cu") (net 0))
 (segment (start 88.8 46.8) (end 87.7 47.9) (width 0.2) (layer "B.Cu") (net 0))
 (segment (start 105.2 49.2) (end 108.2 52.2) (width 0.25) (layer "B.Cu") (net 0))
 (segment (start 101.5 58.5) (end 101.5 60.5) (width 0.2) (layer "B.Cu") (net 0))
 (segment (start 101.2 64.6) (end 102.6 64.6) (width 0.2) (layer "B.Cu") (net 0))
 (segment (start 104.6 49.2) (end 105.2 49.2) (width 0.25) (layer "B.Cu") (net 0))
 (segment (start 102 55.9) (end 100.8 57.1) (width 0.2) (layer "B.Cu") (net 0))
 (segment (start 104.6 55.4) (end 106.6 57.4) (width 0.25) (layer "B.Cu") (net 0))
 (segment (start 98.23 58.6) (end 98.2 58.6) (width 0.2) (layer "B.Cu") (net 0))
 (segment (start 118.455 54.345) (end 116.2 52.09) (width 0.2) (layer "B.Cu") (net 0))
 (segment (start 88.1 52.130127) (end 87 51.030127) (width 0.2) (layer "B.Cu") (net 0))
 (segment (start 98.6 63.11) (end 97.11 63.11) (width 0.2) (layer "B.Cu") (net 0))
 (segment (start 121.8 61.8) (end 121.8 55.2) (width 0.2) (layer "B.Cu") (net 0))
 (segment (start 101.5 60.5) (end 99.6 62.4) (width 0.2) (layer "B.Cu") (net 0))
 (segment (start 103.2 62.8) (end 103.2 64) (width 0.2) (layer "B.Cu") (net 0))
 (segment (start 98.8 61.6) (end 98.4 61.6) (width 0.2) (layer "B.Cu") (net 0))
 (segment (start 98.2 58.6) (end 97.2 57.6) (width 0.2) (layer "B.Cu") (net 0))
 (segment (start 103.05 56.95) (end 101.5 58.5) (width 0.2) (layer "B.Cu") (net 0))
 (segment (start 101.64 53.71) (end 101.64 52.16) (width 0.25) (layer "B.Cu") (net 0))
 (segment (start 116 57.6) (end 116 60.997812) (width 0.2) (layer "B.Cu") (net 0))
 (segment (start 108.2 52.2) (end 110.6 52.2) (width 0.25) (layer "B.Cu") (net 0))
 (segment (start 118.93125 59.933438) (end 118.455 59.457188) (width 0.2) (layer "B.Cu") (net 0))
 (segment (start 88.6 47.8) (end 88.8 47.6) (width 0.2) (layer "B.Cu") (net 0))
 (segment (start 102.95 59) (end 102.95 58.05) (width 0.2) (layer "B.Cu") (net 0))
 (segment (start 109.8 66.6) (end 109.8 58.6) (width 0.2) (layer "B.Cu") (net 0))
 (segment (start 98.6 63.11) (end 100.09 64.6) (width 0.2) (layer "B.Cu") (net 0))
 (segment (start 121.8 55.2) (end 118.879664 52.279664) (width 0.2) (layer "B.Cu") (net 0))
 (segment (start 107.63 55.6) (end 108.6 55.6) (width 0.2) (layer "B.Cu") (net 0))
 (segment (start 119.4 64.2) (end 121.8 61.8) (width 0.2) (layer "B.Cu") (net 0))
 (segment (start 98.23 58.6) (end 98.94 59.31) (width 0.2) (layer "B.Cu") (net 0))
 (segment (start 118.455 51.644696) (end 118.879664 51.220032) (width 0.2) (layer "B.Cu") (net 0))
 (segment (start 100.8 59.6) (end 98.8 61.6) (width 0.2) (layer "B.Cu") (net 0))
 (segment (start 88.657611 49.453084) (end 88.83802 49.453084) (width 0.2) (layer "B.Cu") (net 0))
 (segment (start 106.6 44.6) (end 109.2 47.2) (width 0.2) (layer "B.Cu") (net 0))
 (segment (start 98.4 61.6) (end 94.6 57.8) (width 0.2) (layer "B.Cu") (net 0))
 (segment (start 87.7 47.9) (end 91 44.6) (width 0.2) (layer "B.Cu") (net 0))
 (segment (start 101.165 62.735) (end 100.79 63.11) (width 0.2) (layer "B.Cu") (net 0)))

